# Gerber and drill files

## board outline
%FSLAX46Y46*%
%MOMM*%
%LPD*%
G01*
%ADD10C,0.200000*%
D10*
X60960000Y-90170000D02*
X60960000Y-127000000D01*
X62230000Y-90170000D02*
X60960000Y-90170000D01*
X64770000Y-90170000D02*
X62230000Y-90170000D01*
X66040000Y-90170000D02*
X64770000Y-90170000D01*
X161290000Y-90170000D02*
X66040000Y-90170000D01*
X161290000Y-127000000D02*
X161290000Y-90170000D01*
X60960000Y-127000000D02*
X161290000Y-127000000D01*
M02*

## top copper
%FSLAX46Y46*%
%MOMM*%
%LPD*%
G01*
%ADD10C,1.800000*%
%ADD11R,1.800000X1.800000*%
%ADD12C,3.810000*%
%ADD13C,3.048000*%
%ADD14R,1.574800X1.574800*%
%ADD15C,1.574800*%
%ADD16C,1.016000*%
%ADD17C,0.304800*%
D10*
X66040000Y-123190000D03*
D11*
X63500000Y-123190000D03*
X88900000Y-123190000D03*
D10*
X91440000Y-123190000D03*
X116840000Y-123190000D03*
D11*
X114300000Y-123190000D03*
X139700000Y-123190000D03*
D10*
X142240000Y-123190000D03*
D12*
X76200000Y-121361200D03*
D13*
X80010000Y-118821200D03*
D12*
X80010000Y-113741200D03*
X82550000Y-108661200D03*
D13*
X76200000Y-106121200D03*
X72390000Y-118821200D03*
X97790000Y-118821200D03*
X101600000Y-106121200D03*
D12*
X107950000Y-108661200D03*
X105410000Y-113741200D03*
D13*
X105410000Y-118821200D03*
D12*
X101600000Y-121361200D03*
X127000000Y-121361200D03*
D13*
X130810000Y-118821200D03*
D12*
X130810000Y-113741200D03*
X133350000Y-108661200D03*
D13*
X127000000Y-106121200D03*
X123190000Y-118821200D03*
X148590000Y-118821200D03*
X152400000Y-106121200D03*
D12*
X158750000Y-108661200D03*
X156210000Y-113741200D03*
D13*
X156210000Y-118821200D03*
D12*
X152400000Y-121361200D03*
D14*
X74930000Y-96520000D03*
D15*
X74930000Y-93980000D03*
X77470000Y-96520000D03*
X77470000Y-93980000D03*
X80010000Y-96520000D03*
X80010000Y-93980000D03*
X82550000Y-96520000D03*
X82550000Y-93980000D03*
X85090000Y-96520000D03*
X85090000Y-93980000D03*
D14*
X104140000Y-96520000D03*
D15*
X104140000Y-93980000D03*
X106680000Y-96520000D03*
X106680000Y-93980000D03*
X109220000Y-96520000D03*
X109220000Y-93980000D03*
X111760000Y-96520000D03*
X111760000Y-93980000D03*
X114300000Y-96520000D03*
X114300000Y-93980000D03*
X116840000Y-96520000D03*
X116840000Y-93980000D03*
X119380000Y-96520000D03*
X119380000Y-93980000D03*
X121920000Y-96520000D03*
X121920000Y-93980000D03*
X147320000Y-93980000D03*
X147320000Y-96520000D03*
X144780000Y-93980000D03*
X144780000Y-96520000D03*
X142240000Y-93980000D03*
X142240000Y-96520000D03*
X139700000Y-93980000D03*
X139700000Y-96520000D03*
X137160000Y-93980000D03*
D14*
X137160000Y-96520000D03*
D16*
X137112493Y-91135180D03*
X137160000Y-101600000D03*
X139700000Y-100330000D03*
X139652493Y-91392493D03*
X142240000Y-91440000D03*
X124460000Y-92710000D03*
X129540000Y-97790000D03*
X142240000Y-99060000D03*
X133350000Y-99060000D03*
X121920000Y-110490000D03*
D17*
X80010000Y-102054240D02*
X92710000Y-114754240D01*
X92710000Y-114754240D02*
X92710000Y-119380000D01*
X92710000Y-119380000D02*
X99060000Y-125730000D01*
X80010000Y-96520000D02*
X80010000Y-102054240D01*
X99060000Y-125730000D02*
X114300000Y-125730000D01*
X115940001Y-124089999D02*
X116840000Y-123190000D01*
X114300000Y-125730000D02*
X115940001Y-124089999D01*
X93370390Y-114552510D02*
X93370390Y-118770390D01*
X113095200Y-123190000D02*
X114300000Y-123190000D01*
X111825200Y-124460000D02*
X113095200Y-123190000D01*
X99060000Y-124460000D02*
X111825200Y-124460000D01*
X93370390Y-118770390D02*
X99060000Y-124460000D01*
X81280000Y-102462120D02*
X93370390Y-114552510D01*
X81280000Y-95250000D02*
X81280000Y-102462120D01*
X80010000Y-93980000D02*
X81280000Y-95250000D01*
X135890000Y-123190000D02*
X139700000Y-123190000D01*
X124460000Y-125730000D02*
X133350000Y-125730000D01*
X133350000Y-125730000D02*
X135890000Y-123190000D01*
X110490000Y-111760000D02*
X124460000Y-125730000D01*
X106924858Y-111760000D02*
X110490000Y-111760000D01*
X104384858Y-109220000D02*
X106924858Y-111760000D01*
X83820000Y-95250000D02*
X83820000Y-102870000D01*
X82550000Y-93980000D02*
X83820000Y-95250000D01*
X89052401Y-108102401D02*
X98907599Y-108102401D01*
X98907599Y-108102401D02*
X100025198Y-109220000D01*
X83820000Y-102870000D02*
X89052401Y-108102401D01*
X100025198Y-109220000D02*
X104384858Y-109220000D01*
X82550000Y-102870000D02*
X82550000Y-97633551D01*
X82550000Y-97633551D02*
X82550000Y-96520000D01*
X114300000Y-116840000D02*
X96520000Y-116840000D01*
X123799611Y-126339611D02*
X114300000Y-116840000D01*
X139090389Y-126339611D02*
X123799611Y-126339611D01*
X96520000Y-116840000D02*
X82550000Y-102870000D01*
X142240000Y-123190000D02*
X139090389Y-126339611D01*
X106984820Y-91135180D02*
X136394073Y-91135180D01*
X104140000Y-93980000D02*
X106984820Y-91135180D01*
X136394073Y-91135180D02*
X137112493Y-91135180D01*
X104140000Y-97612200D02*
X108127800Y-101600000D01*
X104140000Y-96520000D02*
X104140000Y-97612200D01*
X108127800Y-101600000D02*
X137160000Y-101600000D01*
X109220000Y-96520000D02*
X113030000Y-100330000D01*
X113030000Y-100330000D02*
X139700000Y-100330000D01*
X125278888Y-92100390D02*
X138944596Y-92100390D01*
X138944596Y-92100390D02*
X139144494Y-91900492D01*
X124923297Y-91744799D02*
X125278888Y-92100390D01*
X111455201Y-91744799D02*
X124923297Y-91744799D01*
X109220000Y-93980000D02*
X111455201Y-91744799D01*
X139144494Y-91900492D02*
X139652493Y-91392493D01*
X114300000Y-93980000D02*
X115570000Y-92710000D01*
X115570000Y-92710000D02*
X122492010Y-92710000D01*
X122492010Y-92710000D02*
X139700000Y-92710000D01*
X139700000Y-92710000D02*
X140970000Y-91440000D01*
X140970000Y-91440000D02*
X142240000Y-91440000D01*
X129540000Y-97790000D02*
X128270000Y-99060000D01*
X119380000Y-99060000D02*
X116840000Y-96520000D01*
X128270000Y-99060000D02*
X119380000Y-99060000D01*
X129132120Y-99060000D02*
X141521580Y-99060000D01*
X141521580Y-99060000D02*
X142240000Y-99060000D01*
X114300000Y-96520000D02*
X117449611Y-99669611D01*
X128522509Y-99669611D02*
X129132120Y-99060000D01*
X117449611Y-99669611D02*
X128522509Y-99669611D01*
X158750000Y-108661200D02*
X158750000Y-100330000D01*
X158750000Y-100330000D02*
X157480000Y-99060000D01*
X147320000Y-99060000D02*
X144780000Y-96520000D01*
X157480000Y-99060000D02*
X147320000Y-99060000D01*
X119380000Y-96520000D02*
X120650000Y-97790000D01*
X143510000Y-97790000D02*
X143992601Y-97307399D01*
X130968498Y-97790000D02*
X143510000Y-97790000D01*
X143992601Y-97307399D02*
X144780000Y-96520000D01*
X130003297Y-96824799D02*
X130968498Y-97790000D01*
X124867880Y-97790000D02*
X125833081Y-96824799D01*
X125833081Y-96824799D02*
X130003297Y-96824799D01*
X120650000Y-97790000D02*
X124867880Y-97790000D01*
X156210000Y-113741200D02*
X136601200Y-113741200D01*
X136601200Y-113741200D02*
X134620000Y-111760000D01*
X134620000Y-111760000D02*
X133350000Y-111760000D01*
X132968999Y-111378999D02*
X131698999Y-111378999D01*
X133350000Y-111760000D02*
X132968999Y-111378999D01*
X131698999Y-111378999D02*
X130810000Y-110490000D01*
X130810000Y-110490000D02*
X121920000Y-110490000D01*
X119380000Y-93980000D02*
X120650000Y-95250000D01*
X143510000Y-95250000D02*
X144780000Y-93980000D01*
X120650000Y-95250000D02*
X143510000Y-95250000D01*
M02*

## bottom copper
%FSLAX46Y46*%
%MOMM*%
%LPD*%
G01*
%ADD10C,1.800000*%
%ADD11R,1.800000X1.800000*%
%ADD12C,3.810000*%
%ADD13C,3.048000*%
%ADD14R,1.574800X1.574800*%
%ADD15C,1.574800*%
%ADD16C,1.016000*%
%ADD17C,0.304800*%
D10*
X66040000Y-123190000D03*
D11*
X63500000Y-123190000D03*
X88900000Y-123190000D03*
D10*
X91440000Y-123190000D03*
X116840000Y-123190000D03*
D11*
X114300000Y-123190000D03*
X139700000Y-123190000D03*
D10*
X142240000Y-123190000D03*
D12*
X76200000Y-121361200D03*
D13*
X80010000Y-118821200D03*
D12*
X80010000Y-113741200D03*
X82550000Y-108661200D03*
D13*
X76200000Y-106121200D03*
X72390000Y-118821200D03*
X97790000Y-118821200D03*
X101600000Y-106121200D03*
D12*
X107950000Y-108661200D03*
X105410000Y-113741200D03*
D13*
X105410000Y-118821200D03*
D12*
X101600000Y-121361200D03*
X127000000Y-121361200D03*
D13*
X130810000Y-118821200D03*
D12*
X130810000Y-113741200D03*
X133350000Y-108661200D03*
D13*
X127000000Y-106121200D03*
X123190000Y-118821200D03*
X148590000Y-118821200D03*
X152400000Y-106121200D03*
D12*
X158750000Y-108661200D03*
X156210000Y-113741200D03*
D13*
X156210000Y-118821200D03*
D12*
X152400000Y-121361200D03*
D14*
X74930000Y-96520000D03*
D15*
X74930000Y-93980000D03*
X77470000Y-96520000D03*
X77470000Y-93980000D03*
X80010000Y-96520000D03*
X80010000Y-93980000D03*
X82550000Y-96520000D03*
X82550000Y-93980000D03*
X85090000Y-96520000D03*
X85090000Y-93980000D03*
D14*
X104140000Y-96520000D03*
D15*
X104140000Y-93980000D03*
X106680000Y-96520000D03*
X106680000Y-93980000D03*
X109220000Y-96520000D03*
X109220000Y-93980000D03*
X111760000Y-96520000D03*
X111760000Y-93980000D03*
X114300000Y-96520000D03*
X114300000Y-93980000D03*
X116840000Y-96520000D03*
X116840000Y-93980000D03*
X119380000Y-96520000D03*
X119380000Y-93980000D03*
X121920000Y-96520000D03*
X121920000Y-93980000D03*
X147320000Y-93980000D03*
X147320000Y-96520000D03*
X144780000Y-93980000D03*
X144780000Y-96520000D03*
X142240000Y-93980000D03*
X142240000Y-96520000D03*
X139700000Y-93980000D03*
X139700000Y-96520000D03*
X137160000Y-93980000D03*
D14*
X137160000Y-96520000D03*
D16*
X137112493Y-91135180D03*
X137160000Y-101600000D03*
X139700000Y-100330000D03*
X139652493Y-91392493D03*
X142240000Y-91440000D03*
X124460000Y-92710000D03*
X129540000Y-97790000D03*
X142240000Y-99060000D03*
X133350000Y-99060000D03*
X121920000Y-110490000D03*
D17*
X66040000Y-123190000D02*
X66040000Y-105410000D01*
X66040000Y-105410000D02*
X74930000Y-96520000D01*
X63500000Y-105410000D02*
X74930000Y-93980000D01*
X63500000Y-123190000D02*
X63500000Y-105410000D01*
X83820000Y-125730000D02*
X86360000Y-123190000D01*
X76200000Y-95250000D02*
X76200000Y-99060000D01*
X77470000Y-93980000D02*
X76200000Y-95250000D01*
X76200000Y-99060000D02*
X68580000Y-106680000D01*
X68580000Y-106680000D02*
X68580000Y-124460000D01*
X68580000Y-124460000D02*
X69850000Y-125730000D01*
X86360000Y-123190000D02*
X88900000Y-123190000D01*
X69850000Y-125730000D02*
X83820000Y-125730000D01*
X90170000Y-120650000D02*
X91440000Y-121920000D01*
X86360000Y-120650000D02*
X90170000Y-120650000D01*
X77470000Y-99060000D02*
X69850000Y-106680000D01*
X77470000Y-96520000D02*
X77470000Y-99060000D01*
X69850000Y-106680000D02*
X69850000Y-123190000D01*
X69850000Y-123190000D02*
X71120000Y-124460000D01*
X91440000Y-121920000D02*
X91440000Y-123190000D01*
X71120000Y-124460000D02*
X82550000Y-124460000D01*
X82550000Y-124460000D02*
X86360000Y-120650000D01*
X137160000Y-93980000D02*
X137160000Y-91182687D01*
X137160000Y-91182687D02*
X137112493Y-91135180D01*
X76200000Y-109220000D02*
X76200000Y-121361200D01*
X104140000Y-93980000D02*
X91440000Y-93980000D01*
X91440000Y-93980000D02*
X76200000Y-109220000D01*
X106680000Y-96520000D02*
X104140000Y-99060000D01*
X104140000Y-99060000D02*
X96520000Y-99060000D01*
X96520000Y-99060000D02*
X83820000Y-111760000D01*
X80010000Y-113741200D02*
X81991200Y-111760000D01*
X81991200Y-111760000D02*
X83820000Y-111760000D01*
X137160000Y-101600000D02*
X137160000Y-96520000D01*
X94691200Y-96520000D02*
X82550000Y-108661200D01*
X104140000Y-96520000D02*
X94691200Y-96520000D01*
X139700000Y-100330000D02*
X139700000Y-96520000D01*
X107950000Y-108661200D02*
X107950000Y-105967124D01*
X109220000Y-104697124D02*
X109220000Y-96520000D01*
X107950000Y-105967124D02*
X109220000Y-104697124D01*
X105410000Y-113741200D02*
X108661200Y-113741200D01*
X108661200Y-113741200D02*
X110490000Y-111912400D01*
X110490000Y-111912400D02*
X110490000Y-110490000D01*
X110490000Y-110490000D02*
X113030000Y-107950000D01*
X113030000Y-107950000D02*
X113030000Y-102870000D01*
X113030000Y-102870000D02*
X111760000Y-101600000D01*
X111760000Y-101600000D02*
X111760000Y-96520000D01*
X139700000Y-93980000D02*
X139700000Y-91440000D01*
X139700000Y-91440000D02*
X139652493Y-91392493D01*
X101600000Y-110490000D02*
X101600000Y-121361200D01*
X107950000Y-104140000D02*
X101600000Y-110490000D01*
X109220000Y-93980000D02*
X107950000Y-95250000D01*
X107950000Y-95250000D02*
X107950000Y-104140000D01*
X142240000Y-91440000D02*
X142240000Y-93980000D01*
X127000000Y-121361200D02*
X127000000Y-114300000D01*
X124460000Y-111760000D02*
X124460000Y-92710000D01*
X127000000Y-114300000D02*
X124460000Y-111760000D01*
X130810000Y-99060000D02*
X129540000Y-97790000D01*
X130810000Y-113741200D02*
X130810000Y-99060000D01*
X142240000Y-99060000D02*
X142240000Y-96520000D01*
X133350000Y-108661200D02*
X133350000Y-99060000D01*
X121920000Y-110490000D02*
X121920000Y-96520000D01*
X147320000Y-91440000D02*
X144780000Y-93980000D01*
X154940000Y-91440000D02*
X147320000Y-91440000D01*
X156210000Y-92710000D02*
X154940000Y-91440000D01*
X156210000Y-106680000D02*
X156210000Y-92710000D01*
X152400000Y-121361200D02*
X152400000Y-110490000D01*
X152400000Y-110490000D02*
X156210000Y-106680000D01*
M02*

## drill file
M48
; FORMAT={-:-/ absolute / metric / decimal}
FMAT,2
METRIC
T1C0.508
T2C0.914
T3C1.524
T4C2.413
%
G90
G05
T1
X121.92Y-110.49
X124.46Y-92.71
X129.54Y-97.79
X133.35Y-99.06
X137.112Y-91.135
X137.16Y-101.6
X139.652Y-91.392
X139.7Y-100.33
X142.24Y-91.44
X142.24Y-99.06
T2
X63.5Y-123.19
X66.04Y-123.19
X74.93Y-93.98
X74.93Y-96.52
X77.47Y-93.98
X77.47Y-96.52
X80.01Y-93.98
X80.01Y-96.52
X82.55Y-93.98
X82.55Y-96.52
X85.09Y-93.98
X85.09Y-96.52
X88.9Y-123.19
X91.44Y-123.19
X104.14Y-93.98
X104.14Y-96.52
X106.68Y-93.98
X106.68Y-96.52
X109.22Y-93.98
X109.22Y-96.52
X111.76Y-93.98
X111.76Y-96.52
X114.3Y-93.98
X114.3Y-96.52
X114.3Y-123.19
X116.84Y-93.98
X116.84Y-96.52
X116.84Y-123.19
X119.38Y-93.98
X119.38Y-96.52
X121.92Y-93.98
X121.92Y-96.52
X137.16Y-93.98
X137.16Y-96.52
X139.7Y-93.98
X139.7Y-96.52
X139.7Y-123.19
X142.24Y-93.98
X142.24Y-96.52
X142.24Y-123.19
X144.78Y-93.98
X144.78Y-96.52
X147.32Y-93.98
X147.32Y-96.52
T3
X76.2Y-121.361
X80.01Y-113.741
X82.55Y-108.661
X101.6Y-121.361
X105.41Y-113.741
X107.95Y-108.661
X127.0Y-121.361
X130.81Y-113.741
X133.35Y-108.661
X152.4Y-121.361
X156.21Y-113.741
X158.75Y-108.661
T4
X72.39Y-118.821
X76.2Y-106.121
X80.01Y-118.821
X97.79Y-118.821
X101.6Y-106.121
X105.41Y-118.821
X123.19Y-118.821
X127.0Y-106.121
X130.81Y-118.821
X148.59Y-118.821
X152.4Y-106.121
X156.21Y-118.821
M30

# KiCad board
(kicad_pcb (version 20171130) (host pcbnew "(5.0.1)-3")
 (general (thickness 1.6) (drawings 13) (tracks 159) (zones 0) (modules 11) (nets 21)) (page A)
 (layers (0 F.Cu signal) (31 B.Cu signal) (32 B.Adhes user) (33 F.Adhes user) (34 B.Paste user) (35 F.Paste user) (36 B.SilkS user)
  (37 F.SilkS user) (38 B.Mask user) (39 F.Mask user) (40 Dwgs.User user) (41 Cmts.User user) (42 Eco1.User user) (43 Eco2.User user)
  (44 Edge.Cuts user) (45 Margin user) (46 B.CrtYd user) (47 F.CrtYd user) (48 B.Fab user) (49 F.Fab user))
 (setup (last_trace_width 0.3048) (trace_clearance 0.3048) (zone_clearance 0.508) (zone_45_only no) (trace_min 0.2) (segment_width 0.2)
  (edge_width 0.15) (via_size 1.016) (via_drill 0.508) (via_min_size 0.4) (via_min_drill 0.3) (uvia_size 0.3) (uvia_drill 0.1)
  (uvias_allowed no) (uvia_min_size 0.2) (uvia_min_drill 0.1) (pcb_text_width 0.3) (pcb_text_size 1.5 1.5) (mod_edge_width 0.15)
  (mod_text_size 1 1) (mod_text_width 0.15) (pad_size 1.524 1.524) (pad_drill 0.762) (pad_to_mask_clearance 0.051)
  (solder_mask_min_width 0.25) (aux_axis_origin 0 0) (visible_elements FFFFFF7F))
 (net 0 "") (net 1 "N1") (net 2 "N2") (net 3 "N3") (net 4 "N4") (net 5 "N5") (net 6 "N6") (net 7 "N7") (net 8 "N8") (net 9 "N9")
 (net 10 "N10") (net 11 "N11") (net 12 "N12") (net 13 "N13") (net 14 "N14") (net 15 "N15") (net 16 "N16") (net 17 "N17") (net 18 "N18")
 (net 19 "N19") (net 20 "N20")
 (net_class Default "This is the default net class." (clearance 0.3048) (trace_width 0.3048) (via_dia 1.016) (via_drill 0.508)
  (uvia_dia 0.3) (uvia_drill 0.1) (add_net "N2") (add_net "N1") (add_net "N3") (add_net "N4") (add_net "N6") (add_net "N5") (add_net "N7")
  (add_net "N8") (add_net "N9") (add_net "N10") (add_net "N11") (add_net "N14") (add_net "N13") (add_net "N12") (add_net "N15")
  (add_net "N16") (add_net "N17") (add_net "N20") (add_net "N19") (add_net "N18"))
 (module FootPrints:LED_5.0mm (layer F.Cu) (at 63.5 123.19)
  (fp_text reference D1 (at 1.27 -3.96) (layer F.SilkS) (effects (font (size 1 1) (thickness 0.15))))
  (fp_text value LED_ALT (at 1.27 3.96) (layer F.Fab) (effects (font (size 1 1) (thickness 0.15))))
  (pad 2 thru_hole circle (at 2.54 0) (size 1.8 1.8) (drill 0.9144) (layers *.Cu *.Mask) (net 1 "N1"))
  (pad 1 thru_hole rect (at 0 0) (size 1.8 1.8) (drill 0.9144) (layers *.Cu *.Mask) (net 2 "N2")))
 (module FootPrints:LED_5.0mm (layer F.Cu) (at 88.9 123.19)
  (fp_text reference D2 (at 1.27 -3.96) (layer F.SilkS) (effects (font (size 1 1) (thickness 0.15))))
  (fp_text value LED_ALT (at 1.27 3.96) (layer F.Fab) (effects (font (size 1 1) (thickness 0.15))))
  (pad 1 thru_hole rect (at 0 0) (size 1.8 1.8) (drill 0.9144) (layers *.Cu *.Mask) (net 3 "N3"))
  (pad 2 thru_hole circle (at 2.54 0) (size 1.8 1.8) (drill 0.9144) (layers *.Cu *.Mask) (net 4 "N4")))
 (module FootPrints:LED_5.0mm (layer F.Cu) (at 114.3 123.19)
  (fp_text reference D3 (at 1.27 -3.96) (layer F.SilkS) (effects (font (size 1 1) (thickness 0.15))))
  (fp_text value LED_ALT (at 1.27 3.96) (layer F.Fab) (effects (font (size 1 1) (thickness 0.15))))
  (pad 2 thru_hole circle (at 2.54 0) (size 1.8 1.8) (drill 0.9144) (layers *.Cu *.Mask) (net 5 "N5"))
  (pad 1 thru_hole rect (at 0 0) (size 1.8 1.8) (drill 0.9144) (layers *.Cu *.Mask) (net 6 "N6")))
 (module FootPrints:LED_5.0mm (layer F.Cu) (at 139.7 123.19)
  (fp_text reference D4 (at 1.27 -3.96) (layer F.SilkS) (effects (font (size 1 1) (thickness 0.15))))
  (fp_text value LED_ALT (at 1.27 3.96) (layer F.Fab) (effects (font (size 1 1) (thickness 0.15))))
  (pad 1 thru_hole rect (at 0 0) (size 1.8 1.8) (drill 0.9144) (layers *.Cu *.Mask) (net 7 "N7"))
  (pad 2 thru_hole circle (at 2.54 0) (size 1.8 1.8) (drill 0.9144) (layers *.Cu *.Mask) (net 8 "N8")))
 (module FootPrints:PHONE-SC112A (layer F.Cu) (at 76.2 127 270)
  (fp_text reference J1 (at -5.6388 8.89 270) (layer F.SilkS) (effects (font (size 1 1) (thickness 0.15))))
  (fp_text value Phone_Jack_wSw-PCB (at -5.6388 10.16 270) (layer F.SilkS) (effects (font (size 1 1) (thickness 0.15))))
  (pad 1 thru_hole circle (at -5.6388 0 270) (size 3.81 3.81) (drill 1.524) (layers *.Cu *.Mask F.SilkS) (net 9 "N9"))
  (pad "" thru_hole circle (at -8.1788 -3.81 270) (size 3.048 3.048) (drill 2.413) (layers *.Cu *.Mask F.SilkS))
  (pad 2 thru_hole circle (at -13.2588 -3.81 270) (size 3.81 3.81) (drill 1.524) (layers *.Cu *.Mask F.SilkS) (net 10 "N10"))
  (pad 3 thru_hole circle (at -18.3388 -6.35 270) (size 3.81 3.81) (drill 1.524) (layers *.Cu *.Mask F.SilkS) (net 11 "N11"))
  (pad "" thru_hole circle (at -20.8788 0 270) (size 3.048 3.048) (drill 2.413) (layers *.Cu *.Mask F.SilkS))
  (pad "" thru_hole circle (at -8.1788 3.81 270) (size 3.048 3.048) (drill 2.413) (layers *.Cu *.Mask F.SilkS)))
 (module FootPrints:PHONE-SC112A (layer F.Cu) (at 101.6 127 270)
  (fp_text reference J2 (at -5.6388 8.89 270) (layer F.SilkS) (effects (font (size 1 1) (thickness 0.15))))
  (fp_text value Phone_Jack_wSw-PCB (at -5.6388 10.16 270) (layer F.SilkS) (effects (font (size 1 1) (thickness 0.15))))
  (pad "" thru_hole circle (at -8.1788 3.81 270) (size 3.048 3.048) (drill 2.413) (layers *.Cu *.Mask F.SilkS))
  (pad "" thru_hole circle (at -20.8788 0 270) (size 3.048 3.048) (drill 2.413) (layers *.Cu *.Mask F.SilkS))
  (pad 3 thru_hole circle (at -18.3388 -6.35 270) (size 3.81 3.81) (drill 1.524) (layers *.Cu *.Mask F.SilkS) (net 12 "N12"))
  (pad 2 thru_hole circle (at -13.2588 -3.81 270) (size 3.81 3.81) (drill 1.524) (layers *.Cu *.Mask F.SilkS) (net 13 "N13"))
  (pad "" thru_hole circle (at -8.1788 -3.81 270) (size 3.048 3.048) (drill 2.413) (layers *.Cu *.Mask F.SilkS))
  (pad 1 thru_hole circle (at -5.6388 0 270) (size 3.81 3.81) (drill 1.524) (layers *.Cu *.Mask F.SilkS) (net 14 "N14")))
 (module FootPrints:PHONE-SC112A (layer F.Cu) (at 127 127 270)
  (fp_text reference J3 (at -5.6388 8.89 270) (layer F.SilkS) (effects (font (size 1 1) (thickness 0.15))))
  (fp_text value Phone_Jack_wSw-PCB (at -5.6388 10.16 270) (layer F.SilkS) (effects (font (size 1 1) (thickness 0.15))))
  (pad 1 thru_hole circle (at -5.6388 0 270) (size 3.81 3.81) (drill 1.524) (layers *.Cu *.Mask F.SilkS) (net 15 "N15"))
  (pad "" thru_hole circle (at -8.1788 -3.81 270) (size 3.048 3.048) (drill 2.413) (layers *.Cu *.Mask F.SilkS))
  (pad 2 thru_hole circle (at -13.2588 -3.81 270) (size 3.81 3.81) (drill 1.524) (layers *.Cu *.Mask F.SilkS) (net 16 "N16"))
  (pad 3 thru_hole circle (at -18.3388 -6.35 270) (size 3.81 3.81) (drill 1.524) (layers *.Cu *.Mask F.SilkS) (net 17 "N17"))
  (pad "" thru_hole circle (at -20.8788 0 270) (size 3.048 3.048) (drill 2.413) (layers *.Cu *.Mask F.SilkS))
  (pad "" thru_hole circle (at -8.1788 3.81 270) (size 3.048 3.048) (drill 2.413) (layers *.Cu *.Mask F.SilkS)))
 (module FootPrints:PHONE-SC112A (layer F.Cu) (at 152.4 127 270)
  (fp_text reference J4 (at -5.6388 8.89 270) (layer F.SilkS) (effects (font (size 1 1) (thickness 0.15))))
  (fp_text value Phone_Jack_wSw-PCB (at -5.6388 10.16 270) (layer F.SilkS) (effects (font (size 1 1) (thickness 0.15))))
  (pad "" thru_hole circle (at -8.1788 3.81 270) (size 3.048 3.048) (drill 2.413) (layers *.Cu *.Mask F.SilkS))
  (pad "" thru_hole circle (at -20.8788 0 270) (size 3.048 3.048) (drill 2.413) (layers *.Cu *.Mask F.SilkS))
  (pad 3 thru_hole circle (at -18.3388 -6.35 270) (size 3.81 3.81) (drill 1.524) (layers *.Cu *.Mask F.SilkS) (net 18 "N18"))
  (pad 2 thru_hole circle (at -13.2588 -3.81 270) (size 3.81 3.81) (drill 1.524) (layers *.Cu *.Mask F.SilkS) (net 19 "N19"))
  (pad "" thru_hole circle (at -8.1788 -3.81 270) (size 3.048 3.048) (drill 2.413) (layers *.Cu *.Mask F.SilkS))
  (pad 1 thru_hole circle (at -5.6388 0 270) (size 3.81 3.81) (drill 1.524) (layers *.Cu *.Mask F.SilkS) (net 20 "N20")))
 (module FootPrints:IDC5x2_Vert (layer F.Cu) (at 80.01 95.25 180)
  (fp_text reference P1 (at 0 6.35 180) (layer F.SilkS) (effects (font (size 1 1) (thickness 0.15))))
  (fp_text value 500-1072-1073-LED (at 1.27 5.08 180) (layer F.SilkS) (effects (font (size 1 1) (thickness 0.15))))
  (pad 1 thru_hole rect (at 5.08 -1.27 180) (size 1.5748 1.5748) (drill 0.9144) (layers *.Cu *.Mask F.SilkS) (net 1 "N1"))
  (pad 2 thru_hole circle (at 5.08 1.27 180) (size 1.5748 1.5748) (drill 0.9144) (layers *.Cu *.Mask F.SilkS) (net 2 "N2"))
  (pad 3 thru_hole circle (at 2.54 -1.27 180) (size 1.5748 1.5748) (drill 0.9144) (layers *.Cu *.Mask F.SilkS) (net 4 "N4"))
  (pad 4 thru_hole circle (at 2.54 1.27 180) (size 1.5748 1.5748) (drill 0.9144) (layers *.Cu *.Mask F.SilkS) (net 3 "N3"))
  (pad 5 thru_hole circle (at 0 -1.27 180) (size 1.5748 1.5748) (drill 0.9144) (layers *.Cu *.Mask F.SilkS) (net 5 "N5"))
  (pad 6 thru_hole circle (at 0 1.27 180) (size 1.5748 1.5748) (drill 0.9144) (layers *.Cu *.Mask F.SilkS) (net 6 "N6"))
  (pad 7 thru_hole circle (at -2.54 -1.27 180) (size 1.5748 1.5748) (drill 0.9144) (layers *.Cu *.Mask F.SilkS) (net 8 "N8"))
  (pad 8 thru_hole circle (at -2.54 1.27 180) (size 1.5748 1.5748) (drill 0.9144) (layers *.Cu *.Mask F.SilkS) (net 7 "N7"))
  (pad 9 thru_hole circle (at -5.08 -1.27 180) (size 1.5748 1.5748) (drill 0.9144) (layers *.Cu *.Mask F.SilkS))
  (pad 10 thru_hole circle (at -5.08 1.27 180) (size 1.5748 1.5748) (drill 0.9144) (layers *.Cu *.Mask F.SilkS)))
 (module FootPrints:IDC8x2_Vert (layer F.Cu) (at 113.03 95.25 180)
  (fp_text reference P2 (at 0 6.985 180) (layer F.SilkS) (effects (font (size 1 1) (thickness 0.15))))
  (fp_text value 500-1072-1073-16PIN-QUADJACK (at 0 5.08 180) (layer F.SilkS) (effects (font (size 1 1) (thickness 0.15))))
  (pad 1 thru_hole rect (at 8.89 -1.27 180) (size 1.5748 1.5748) (drill 0.9144) (layers *.Cu *.Mask F.SilkS) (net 11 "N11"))
  (pad 2 thru_hole circle (at 8.89 1.27 180) (size 1.5748 1.5748) (drill 0.9144) (layers *.Cu *.Mask F.SilkS) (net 9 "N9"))
  (pad 3 thru_hole circle (at 6.35 -1.27 180) (size 1.5748 1.5748) (drill 0.9144) (layers *.Cu *.Mask F.SilkS) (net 10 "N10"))
  (pad 4 thru_hole circle (at 6.35 1.27 180) (size 1.5748 1.5748) (drill 0.9144) (layers *.Cu *.Mask F.SilkS))
  (pad 5 thru_hole circle (at 3.81 -1.27 180) (size 1.5748 1.5748) (drill 0.9144) (layers *.Cu *.Mask F.SilkS) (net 12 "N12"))
  (pad 6 thru_hole circle (at 3.81 1.27 180) (size 1.5748 1.5748) (drill 0.9144) (layers *.Cu *.Mask F.SilkS) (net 14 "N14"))
  (pad 7 thru_hole circle (at 1.27 -1.27 180) (size 1.5748 1.5748) (drill 0.9144) (layers *.Cu *.Mask F.SilkS) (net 13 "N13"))
  (pad 8 thru_hole circle (at 1.27 1.27 180) (size 1.5748 1.5748) (drill 0.9144) (layers *.Cu *.Mask F.SilkS))
  (pad 9 thru_hole circle (at -1.27 -1.27 180) (size 1.5748 1.5748) (drill 0.9144) (layers *.Cu *.Mask F.SilkS) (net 17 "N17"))
  (pad 10 thru_hole circle (at -1.27 1.27 180) (size 1.5748 1.5748) (drill 0.9144) (layers *.Cu *.Mask F.SilkS) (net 15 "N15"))
  (pad 11 thru_hole circle (at -3.81 -1.27 180) (size 1.5748 1.5748) (drill 0.9144) (layers *.Cu *.Mask F.SilkS) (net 16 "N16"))
  (pad 12 thru_hole circle (at -3.81 1.27 180) (size 1.5748 1.5748) (drill 0.9144) (layers *.Cu *.Mask F.SilkS))
  (pad 13 thru_hole circle (at -6.35 -1.27 180) (size 1.5748 1.5748) (drill 0.9144) (layers *.Cu *.Mask F.SilkS) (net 18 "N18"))
  (pad 14 thru_hole circle (at -6.35 1.27 180) (size 1.5748 1.5748) (drill 0.9144) (layers *.Cu *.Mask F.SilkS) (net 20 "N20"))
  (pad 15 thru_hole circle (at -8.89 -1.27 180) (size 1.5748 1.5748) (drill 0.9144) (layers *.Cu *.Mask F.SilkS) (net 19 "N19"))
  (pad 16 thru_hole circle (at -8.89 1.27 180) (size 1.5748 1.5748) (drill 0.9144) (layers *.Cu *.Mask F.SilkS)))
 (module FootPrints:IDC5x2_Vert (layer F.Cu) (at 142.24 95.25 180)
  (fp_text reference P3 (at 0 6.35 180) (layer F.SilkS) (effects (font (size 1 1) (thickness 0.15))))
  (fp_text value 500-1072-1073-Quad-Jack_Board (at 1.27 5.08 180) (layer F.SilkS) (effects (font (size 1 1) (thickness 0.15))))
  (pad 10 thru_hole circle (at -5.08 1.27 180) (size 1.5748 1.5748) (drill 0.9144) (layers *.Cu *.Mask F.SilkS))
  (pad 9 thru_hole circle (at -5.08 -1.27 180) (size 1.5748 1.5748) (drill 0.9144) (layers *.Cu *.Mask F.SilkS))
  (pad 8 thru_hole circle (at -2.54 1.27 180) (size 1.5748 1.5748) (drill 0.9144) (layers *.Cu *.Mask F.SilkS) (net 20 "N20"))
  (pad 7 thru_hole circle (at -2.54 -1.27 180) (size 1.5748 1.5748) (drill 0.9144) (layers *.Cu *.Mask F.SilkS) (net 18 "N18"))
  (pad 6 thru_hole circle (at 0 1.27 180) (size 1.5748 1.5748) (drill 0.9144) (layers *.Cu *.Mask F.SilkS) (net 15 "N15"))
  (pad 5 thru_hole circle (at 0 -1.27 180) (size 1.5748 1.5748) (drill 0.9144) (layers *.Cu *.Mask F.SilkS) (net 17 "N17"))
  (pad 4 thru_hole circle (at 2.54 1.27 180) (size 1.5748 1.5748) (drill 0.9144) (layers *.Cu *.Mask F.SilkS) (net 14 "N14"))
  (pad 3 thru_hole circle (at 2.54 -1.27 180) (size 1.5748 1.5748) (drill 0.9144) (layers *.Cu *.Mask F.SilkS) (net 12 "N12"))
  (pad 2 thru_hole circle (at 5.08 1.27 180) (size 1.5748 1.5748) (drill 0.9144) (layers *.Cu *.Mask F.SilkS) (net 9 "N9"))
  (pad 1 thru_hole rect (at 5.08 -1.27 180) (size 1.5748 1.5748) (drill 0.9144) (layers *.Cu *.Mask F.SilkS) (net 11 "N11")))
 (gr_line (start 60.96 90.17) (end 60.96 127) (layer Edge.Cuts) (width 0.2))
 (gr_line (start 62.23 90.17) (end 60.96 90.17) (layer Edge.Cuts) (width 0.2))
 (gr_line (start 64.77 90.17) (end 62.23 90.17) (layer Edge.Cuts) (width 0.2))
 (gr_line (start 66.04 90.17) (end 64.77 90.17) (layer Edge.Cuts) (width 0.2))
 (gr_line (start 161.29 90.17) (end 66.04 90.17) (layer Edge.Cuts) (width 0.2))
 (gr_line (start 161.29 127) (end 161.29 90.17) (layer Edge.Cuts) (width 0.2))
 (gr_line (start 60.96 127) (end 161.29 127) (layer Edge.Cuts) (width 0.2))
 (segment (start 66.04 123.19) (end 66.04 105.41) (width 0.3048) (layer B.Cu) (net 1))
 (segment (start 66.04 105.41) (end 74.93 96.52) (width 0.3048) (layer B.Cu) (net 1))
 (segment (start 63.5 105.41) (end 74.93 93.98) (width 0.3048) (layer B.Cu) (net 2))
 (segment (start 63.5 123.19) (end 63.5 105.41) (width 0.3048) (layer B.Cu) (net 2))
 (segment (start 83.82 125.73) (end 86.36 123.19) (width 0.3048) (layer B.Cu) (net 3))
 (segment (start 76.2 95.25) (end 76.2 99.06) (width 0.3048) (layer B.Cu) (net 3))
 (segment (start 77.47 93.98) (end 76.2 95.25) (width 0.3048) (layer B.Cu) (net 3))
 (segment (start 76.2 99.06) (end 68.58 106.68) (width 0.3048) (layer B.Cu) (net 3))
 (segment (start 68.58 106.68) (end 68.58 124.46) (width 0.3048) (layer B.Cu) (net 3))
 (segment (start 68.58 124.46) (end 69.85 125.73) (width 0.3048) (layer B.Cu) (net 3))
 (segment (start 86.36 123.19) (end 88.9 123.19) (width 0.3048) (layer B.Cu) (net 3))
 (segment (start 69.85 125.73) (end 83.82 125.73) (width 0.3048) (layer B.Cu) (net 3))
 (segment (start 90.17 120.65) (end 91.44 121.92) (width 0.3048) (layer B.Cu) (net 4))
 (segment (start 86.36 120.65) (end 90.17 120.65) (width 0.3048) (layer B.Cu) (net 4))
 (segment (start 77.47 99.06) (end 69.85 106.68) (width 0.3048) (layer B.Cu) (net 4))
 (segment (start 77.47 96.52) (end 77.47 99.06) (width 0.3048) (layer B.Cu) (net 4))
 (segment (start 69.85 106.68) (end 69.85 123.19) (width 0.3048) (layer B.Cu) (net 4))
 (segment (start 69.85 123.19) (end 71.12 124.46) (width 0.3048) (layer B.Cu) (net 4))
 (segment (start 91.44 121.92) (end 91.44 123.19) (width 0.3048) (layer B.Cu) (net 4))
 (segment (start 71.12 124.46) (end 82.55 124.46) (width 0.3048) (layer B.Cu) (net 4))
 (segment (start 82.55 124.46) (end 86.36 120.65) (width 0.3048) (layer B.Cu) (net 4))
 (segment (start 80.01 102.05424) (end 92.71 114.75424) (width 0.3048) (layer F.Cu) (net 5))
 (segment (start 92.71 114.75424) (end 92.71 119.38) (width 0.3048) (layer F.Cu) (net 5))
 (segment (start 92.71 119.38) (end 99.06 125.73) (width 0.3048) (layer F.Cu) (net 5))
 (segment (start 80.01 96.52) (end 80.01 102.05424) (width 0.3048) (layer F.Cu) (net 5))
 (segment (start 99.06 125.73) (end 114.3 125.73) (width 0.3048) (layer F.Cu) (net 5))
 (segment (start 115.940001 124.089999) (end 116.84 123.19) (width 0.3048) (layer F.Cu) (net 5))
 (segment (start 114.3 125.73) (end 115.940001 124.089999) (width 0.3048) (layer F.Cu) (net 5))
 (segment (start 93.37039 114.55251) (end 93.37039 118.77039) (width 0.3048) (layer F.Cu) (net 6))
 (segment (start 113.0952 123.19) (end 114.3 123.19) (width 0.3048) (layer F.Cu) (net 6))
 (segment (start 111.8252 124.46) (end 113.0952 123.19) (width 0.3048) (layer F.Cu) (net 6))
 (segment (start 99.06 124.46) (end 111.8252 124.46) (width 0.3048) (layer F.Cu) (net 6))
 (segment (start 93.37039 118.77039) (end 99.06 124.46) (width 0.3048) (layer F.Cu) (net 6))
 (segment (start 81.28 102.46212) (end 93.37039 114.55251) (width 0.3048) (layer F.Cu) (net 6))
 (segment (start 81.28 95.25) (end 81.28 102.46212) (width 0.3048) (layer F.Cu) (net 6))
 (segment (start 80.01 93.98) (end 81.28 95.25) (width 0.3048) (layer F.Cu) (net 6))
 (segment (start 135.89 123.19) (end 139.7 123.19) (width 0.3048) (layer F.Cu) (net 7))
 (segment (start 124.46 125.73) (end 133.35 125.73) (width 0.3048) (layer F.Cu) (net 7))
 (segment (start 133.35 125.73) (end 135.89 123.19) (width 0.3048) (layer F.Cu) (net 7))
 (segment (start 110.49 111.76) (end 124.46 125.73) (width 0.3048) (layer F.Cu) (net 7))
 (segment (start 106.924858 111.76) (end 110.49 111.76) (width 0.3048) (layer F.Cu) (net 7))
 (segment (start 104.384858 109.22) (end 106.924858 111.76) (width 0.3048) (layer F.Cu) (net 7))
 (segment (start 83.82 95.25) (end 83.82 102.87) (width 0.3048) (layer F.Cu) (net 7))
 (segment (start 82.55 93.98) (end 83.82 95.25) (width 0.3048) (layer F.Cu) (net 7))
 (segment (start 89.052401 108.102401) (end 98.907599 108.102401) (width 0.3048) (layer F.Cu) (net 7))
 (segment (start 98.907599 108.102401) (end 100.025198 109.22) (width 0.3048) (layer F.Cu) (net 7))
 (segment (start 83.82 102.87) (end 89.052401 108.102401) (width 0.3048) (layer F.Cu) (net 7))
 (segment (start 100.025198 109.22) (end 104.384858 109.22) (width 0.3048) (layer F.Cu) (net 7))
 (segment (start 82.55 102.87) (end 82.55 97.633551) (width 0.3048) (layer F.Cu) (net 8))
 (segment (start 82.55 97.633551) (end 82.55 96.52) (width 0.3048) (layer F.Cu) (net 8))
 (segment (start 114.3 116.84) (end 96.52 116.84) (width 0.3048) (layer F.Cu) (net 8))
 (segment (start 123.799611 126.339611) (end 114.3 116.84) (width 0.3048) (layer F.Cu) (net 8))
 (segment (start 139.090389 126.339611) (end 123.799611 126.339611) (width 0.3048) (layer F.Cu) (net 8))
 (segment (start 96.52 116.84) (end 82.55 102.87) (width 0.3048) (layer F.Cu) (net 8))
 (segment (start 142.24 123.19) (end 139.090389 126.339611) (width 0.3048) (layer F.Cu) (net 8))
 (segment (start 106.98482 91.13518) (end 136.394073 91.13518) (width 0.3048) (layer F.Cu) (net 9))
 (segment (start 104.14 93.98) (end 106.98482 91.13518) (width 0.3048) (layer F.Cu) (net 9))
 (segment (start 136.394073 91.13518) (end 137.112493 91.13518) (width 0.3048) (layer F.Cu) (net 9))
 (segment (start 137.16 93.98) (end 137.16 91.182687) (width 0.3048) (layer B.Cu) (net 9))
 (segment (start 137.16 91.182687) (end 137.112493 91.13518) (width 0.3048) (layer B.Cu) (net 9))
 (via (at 137.112493 91.13518) (size 1.016) (drill 0.508) (layers F.Cu B.Cu) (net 9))
 (segment (start 76.2 109.22) (end 76.2 121.3612) (width 0.3048) (layer B.Cu) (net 9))
 (segment (start 104.14 93.98) (end 91.44 93.98) (width 0.3048) (layer B.Cu) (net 9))
 (segment (start 91.44 93.98) (end 76.2 109.22) (width 0.3048) (layer B.Cu) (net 9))
 (segment (start 106.68 96.52) (end 104.14 99.06) (width 0.3048) (layer B.Cu) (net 10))
 (segment (start 104.14 99.06) (end 96.52 99.06) (width 0.3048) (layer B.Cu) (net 10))
 (segment (start 96.52 99.06) (end 83.82 111.76) (width 0.3048) (layer B.Cu) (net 10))
 (segment (start 80.01 113.7412) (end 81.9912 111.76) (width 0.3048) (layer B.Cu) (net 10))
 (segment (start 81.9912 111.76) (end 83.82 111.76) (width 0.3048) (layer B.Cu) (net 10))
 (segment (start 104.14 97.6122) (end 108.1278 101.6) (width 0.3048) (layer F.Cu) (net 11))
 (segment (start 104.14 96.52) (end 104.14 97.6122) (width 0.3048) (layer F.Cu) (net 11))
 (via (at 137.16 101.6) (size 1.016) (drill 0.508) (layers F.Cu B.Cu) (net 11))
 (segment (start 108.1278 101.6) (end 137.16 101.6) (width 0.3048) (layer F.Cu) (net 11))
 (segment (start 137.16 101.6) (end 137.16 96.52) (width 0.3048) (layer B.Cu) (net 11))
 (segment (start 94.6912 96.52) (end 82.55 108.6612) (width 0.3048) (layer B.Cu) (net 11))
 (segment (start 104.14 96.52) (end 94.6912 96.52) (width 0.3048) (layer B.Cu) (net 11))
 (segment (start 109.22 96.52) (end 113.03 100.33) (width 0.3048) (layer F.Cu) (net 12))
 (via (at 139.7 100.33) (size 1.016) (drill 0.508) (layers F.Cu B.Cu) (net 12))
 (segment (start 113.03 100.33) (end 139.7 100.33) (width 0.3048) (layer F.Cu) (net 12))
 (segment (start 139.7 100.33) (end 139.7 96.52) (width 0.3048) (layer B.Cu) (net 12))
 (segment (start 107.95 108.6612) (end 107.95 105.967124) (width 0.3048) (layer B.Cu) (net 12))
 (segment (start 109.22 104.697124) (end 109.22 96.52) (width 0.3048) (layer B.Cu) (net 12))
 (segment (start 107.95 105.967124) (end 109.22 104.697124) (width 0.3048) (layer B.Cu) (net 12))
 (segment (start 105.41 113.7412) (end 108.6612 113.7412) (width 0.3048) (layer B.Cu) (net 13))
 (segment (start 108.6612 113.7412) (end 110.49 111.9124) (width 0.3048) (layer B.Cu) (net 13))
 (segment (start 110.49 111.9124) (end 110.49 110.49) (width 0.3048) (layer B.Cu) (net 13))
 (segment (start 110.49 110.49) (end 113.03 107.95) (width 0.3048) (layer B.Cu) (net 13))
 (segment (start 113.03 107.95) (end 113.03 102.87) (width 0.3048) (layer B.Cu) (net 13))
 (segment (start 113.03 102.87) (end 111.76 101.6) (width 0.3048) (layer B.Cu) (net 13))
 (segment (start 111.76 101.6) (end 111.76 96.52) (width 0.3048) (layer B.Cu) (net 13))
 (segment (start 139.7 93.98) (end 139.7 91.44) (width 0.3048) (layer B.Cu) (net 14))
 (via (at 139.652493 91.392493) (size 1.016) (drill 0.508) (layers F.Cu B.Cu) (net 14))
 (segment (start 139.7 91.44) (end 139.652493 91.392493) (width 0.3048) (layer B.Cu) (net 14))
 (segment (start 101.6 110.49) (end 101.6 121.3612) (width 0.3048) (layer B.Cu) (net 14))
 (segment (start 107.95 104.14) (end 101.6 110.49) (width 0.3048) (layer B.Cu) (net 14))
 (segment (start 109.22 93.98) (end 107.95 95.25) (width 0.3048) (layer B.Cu) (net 14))
 (segment (start 107.95 95.25) (end 107.95 104.14) (width 0.3048) (layer B.Cu) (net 14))
 (segment (start 125.278888 92.10039) (end 138.944596 92.10039) (width 0.3048) (layer F.Cu) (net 14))
 (segment (start 138.944596 92.10039) (end 139.144494 91.900492) (width 0.3048) (layer F.Cu) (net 14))
 (segment (start 124.923297 91.744799) (end 125.278888 92.10039) (width 0.3048) (layer F.Cu) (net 14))
 (segment (start 111.455201 91.744799) (end 124.923297 91.744799) (width 0.3048) (layer F.Cu) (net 14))
 (segment (start 109.22 93.98) (end 111.455201 91.744799) (width 0.3048) (layer F.Cu) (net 14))
 (segment (start 139.144494 91.900492) (end 139.652493 91.392493) (width 0.3048) (layer F.Cu) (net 14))
 (segment (start 114.3 93.98) (end 115.57 92.71) (width 0.3048) (layer F.Cu) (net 15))
 (segment (start 115.57 92.71) (end 122.49201 92.71) (width 0.3048) (layer F.Cu) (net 15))
 (segment (start 122.49201 92.71) (end 139.7 92.71) (width 0.3048) (layer F.Cu) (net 15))
 (via (at 142.24 91.44) (size 1.016) (drill 0.508) (layers F.Cu B.Cu) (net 15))
 (segment (start 139.7 92.71) (end 140.97 91.44) (width 0.3048) (layer F.Cu) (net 15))
 (segment (start 140.97 91.44) (end 142.24 91.44) (width 0.3048) (layer F.Cu) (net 15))
 (segment (start 142.24 91.44) (end 142.24 93.98) (width 0.3048) (layer B.Cu) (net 15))
 (segment (start 127 121.3612) (end 127 114.3) (width 0.3048) (layer B.Cu) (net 15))
 (segment (start 124.46 111.76) (end 124.46 92.71) (width 0.3048) (layer B.Cu) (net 15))
 (segment (start 127 114.3) (end 124.46 111.76) (width 0.3048) (layer B.Cu) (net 15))
 (via (at 124.46 92.71) (size 1.016) (drill 0.508) (layers F.Cu B.Cu) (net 15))
 (segment (start 130.81 99.06) (end 129.54 97.79) (width 0.3048) (layer B.Cu) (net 16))
 (via (at 129.54 97.79) (size 1.016) (drill 0.508) (layers F.Cu B.Cu) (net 16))
 (segment (start 130.81 113.7412) (end 130.81 99.06) (width 0.3048) (layer B.Cu) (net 16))
 (segment (start 129.54 97.79) (end 128.27 99.06) (width 0.3048) (layer F.Cu) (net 16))
 (segment (start 119.38 99.06) (end 116.84 96.52) (width 0.3048) (layer F.Cu) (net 16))
 (segment (start 128.27 99.06) (end 119.38 99.06) (width 0.3048) (layer F.Cu) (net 16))
 (via (at 142.24 99.06) (size 1.016) (drill 0.508) (layers F.Cu B.Cu) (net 17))
 (segment (start 142.24 99.06) (end 142.24 96.52) (width 0.3048) (layer B.Cu) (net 17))
 (via (at 133.35 99.06) (size 1.016) (drill 0.508) (layers F.Cu B.Cu) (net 17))
 (segment (start 133.35 108.6612) (end 133.35 99.06) (width 0.3048) (layer B.Cu) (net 17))
 (segment (start 129.13212 99.06) (end 141.52158 99.06) (width 0.3048) (layer F.Cu) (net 17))
 (segment (start 141.52158 99.06) (end 142.24 99.06) (width 0.3048) (layer F.Cu) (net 17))
 (segment (start 114.3 96.52) (end 117.449611 99.669611) (width 0.3048) (layer F.Cu) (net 17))
 (segment (start 128.522509 99.669611) (end 129.13212 99.06) (width 0.3048) (layer F.Cu) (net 17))
 (segment (start 117.449611 99.669611) (end 128.522509 99.669611) (width 0.3048) (layer F.Cu) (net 17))
 (segment (start 158.75 108.6612) (end 158.75 100.33) (width 0.3048) (layer F.Cu) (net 18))
 (segment (start 158.75 100.33) (end 157.48 99.06) (width 0.3048) (layer F.Cu) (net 18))
 (segment (start 147.32 99.06) (end 144.78 96.52) (width 0.3048) (layer F.Cu) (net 18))
 (segment (start 157.48 99.06) (end 147.32 99.06) (width 0.3048) (layer F.Cu) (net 18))
 (segment (start 119.38 96.52) (end 120.65 97.79) (width 0.3048) (layer F.Cu) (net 18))
 (segment (start 143.51 97.79) (end 143.992601 97.307399) (width 0.3048) (layer F.Cu) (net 18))
 (segment (start 130.968498 97.79) (end 143.51 97.79) (width 0.3048) (layer F.Cu) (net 18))
 (segment (start 143.992601 97.307399) (end 144.78 96.52) (width 0.3048) (layer F.Cu) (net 18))
 (segment (start 130.003297 96.824799) (end 130.968498 97.79) (width 0.3048) (layer F.Cu) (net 18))
 (segment (start 124.86788 97.79) (end 125.833081 96.824799) (width 0.3048) (layer F.Cu) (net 18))
 (segment (start 125.833081 96.824799) (end 130.003297 96.824799) (width 0.3048) (layer F.Cu) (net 18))
 (segment (start 120.65 97.79) (end 124.86788 97.79) (width 0.3048) (layer F.Cu) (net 18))
 (segment (start 156.21 113.7412) (end 136.6012 113.7412) (width 0.3048) (layer F.Cu) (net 19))
 (segment (start 136.6012 113.7412) (end 134.62 111.76) (width 0.3048) (layer F.Cu) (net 19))
 (segment (start 134.62 111.76) (end 133.35 111.76) (width 0.3048) (layer F.Cu) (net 19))
 (segment (start 132.968999 111.378999) (end 131.698999 111.378999) (width 0.3048) (layer F.Cu) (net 19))
 (segment (start 133.35 111.76) (end 132.968999 111.378999) (width 0.3048) (layer F.Cu) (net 19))
 (segment (start 131.698999 111.378999) (end 130.81 110.49) (width 0.3048) (layer F.Cu) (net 19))
 (via (at 121.92 110.49) (size 1.016) (drill 0.508) (layers F.Cu B.Cu) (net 19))
 (segment (start 130.81 110.49) (end 121.92 110.49) (width 0.3048) (layer F.Cu) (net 19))
 (segment (start 121.92 110.49) (end 121.92 96.52) (width 0.3048) (layer B.Cu) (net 19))
 (segment (start 119.38 93.98) (end 120.65 95.25) (width 0.3048) (layer F.Cu) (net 20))
 (segment (start 143.51 95.25) (end 144.78 93.98) (width 0.3048) (layer F.Cu) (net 20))
 (segment (start 120.65 95.25) (end 143.51 95.25) (width 0.3048) (layer F.Cu) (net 20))
 (segment (start 147.32 91.44) (end 144.78 93.98) (width 0.3048) (layer B.Cu) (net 20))
 (segment (start 154.94 91.44) (end 147.32 91.44) (width 0.3048) (layer B.Cu) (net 20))
 (segment (start 156.21 92.71) (end 154.94 91.44) (width 0.3048) (layer B.Cu) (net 20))
 (segment (start 156.21 106.68) (end 156.21 92.71) (width 0.3048) (layer B.Cu) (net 20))
 (segment (start 152.4 121.3612) (end 152.4 110.49) (width 0.3048) (layer B.Cu) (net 20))
 (segment (start 152.4 110.49) (end 156.21 106.68) (width 0.3048) (layer B.Cu) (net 20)))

